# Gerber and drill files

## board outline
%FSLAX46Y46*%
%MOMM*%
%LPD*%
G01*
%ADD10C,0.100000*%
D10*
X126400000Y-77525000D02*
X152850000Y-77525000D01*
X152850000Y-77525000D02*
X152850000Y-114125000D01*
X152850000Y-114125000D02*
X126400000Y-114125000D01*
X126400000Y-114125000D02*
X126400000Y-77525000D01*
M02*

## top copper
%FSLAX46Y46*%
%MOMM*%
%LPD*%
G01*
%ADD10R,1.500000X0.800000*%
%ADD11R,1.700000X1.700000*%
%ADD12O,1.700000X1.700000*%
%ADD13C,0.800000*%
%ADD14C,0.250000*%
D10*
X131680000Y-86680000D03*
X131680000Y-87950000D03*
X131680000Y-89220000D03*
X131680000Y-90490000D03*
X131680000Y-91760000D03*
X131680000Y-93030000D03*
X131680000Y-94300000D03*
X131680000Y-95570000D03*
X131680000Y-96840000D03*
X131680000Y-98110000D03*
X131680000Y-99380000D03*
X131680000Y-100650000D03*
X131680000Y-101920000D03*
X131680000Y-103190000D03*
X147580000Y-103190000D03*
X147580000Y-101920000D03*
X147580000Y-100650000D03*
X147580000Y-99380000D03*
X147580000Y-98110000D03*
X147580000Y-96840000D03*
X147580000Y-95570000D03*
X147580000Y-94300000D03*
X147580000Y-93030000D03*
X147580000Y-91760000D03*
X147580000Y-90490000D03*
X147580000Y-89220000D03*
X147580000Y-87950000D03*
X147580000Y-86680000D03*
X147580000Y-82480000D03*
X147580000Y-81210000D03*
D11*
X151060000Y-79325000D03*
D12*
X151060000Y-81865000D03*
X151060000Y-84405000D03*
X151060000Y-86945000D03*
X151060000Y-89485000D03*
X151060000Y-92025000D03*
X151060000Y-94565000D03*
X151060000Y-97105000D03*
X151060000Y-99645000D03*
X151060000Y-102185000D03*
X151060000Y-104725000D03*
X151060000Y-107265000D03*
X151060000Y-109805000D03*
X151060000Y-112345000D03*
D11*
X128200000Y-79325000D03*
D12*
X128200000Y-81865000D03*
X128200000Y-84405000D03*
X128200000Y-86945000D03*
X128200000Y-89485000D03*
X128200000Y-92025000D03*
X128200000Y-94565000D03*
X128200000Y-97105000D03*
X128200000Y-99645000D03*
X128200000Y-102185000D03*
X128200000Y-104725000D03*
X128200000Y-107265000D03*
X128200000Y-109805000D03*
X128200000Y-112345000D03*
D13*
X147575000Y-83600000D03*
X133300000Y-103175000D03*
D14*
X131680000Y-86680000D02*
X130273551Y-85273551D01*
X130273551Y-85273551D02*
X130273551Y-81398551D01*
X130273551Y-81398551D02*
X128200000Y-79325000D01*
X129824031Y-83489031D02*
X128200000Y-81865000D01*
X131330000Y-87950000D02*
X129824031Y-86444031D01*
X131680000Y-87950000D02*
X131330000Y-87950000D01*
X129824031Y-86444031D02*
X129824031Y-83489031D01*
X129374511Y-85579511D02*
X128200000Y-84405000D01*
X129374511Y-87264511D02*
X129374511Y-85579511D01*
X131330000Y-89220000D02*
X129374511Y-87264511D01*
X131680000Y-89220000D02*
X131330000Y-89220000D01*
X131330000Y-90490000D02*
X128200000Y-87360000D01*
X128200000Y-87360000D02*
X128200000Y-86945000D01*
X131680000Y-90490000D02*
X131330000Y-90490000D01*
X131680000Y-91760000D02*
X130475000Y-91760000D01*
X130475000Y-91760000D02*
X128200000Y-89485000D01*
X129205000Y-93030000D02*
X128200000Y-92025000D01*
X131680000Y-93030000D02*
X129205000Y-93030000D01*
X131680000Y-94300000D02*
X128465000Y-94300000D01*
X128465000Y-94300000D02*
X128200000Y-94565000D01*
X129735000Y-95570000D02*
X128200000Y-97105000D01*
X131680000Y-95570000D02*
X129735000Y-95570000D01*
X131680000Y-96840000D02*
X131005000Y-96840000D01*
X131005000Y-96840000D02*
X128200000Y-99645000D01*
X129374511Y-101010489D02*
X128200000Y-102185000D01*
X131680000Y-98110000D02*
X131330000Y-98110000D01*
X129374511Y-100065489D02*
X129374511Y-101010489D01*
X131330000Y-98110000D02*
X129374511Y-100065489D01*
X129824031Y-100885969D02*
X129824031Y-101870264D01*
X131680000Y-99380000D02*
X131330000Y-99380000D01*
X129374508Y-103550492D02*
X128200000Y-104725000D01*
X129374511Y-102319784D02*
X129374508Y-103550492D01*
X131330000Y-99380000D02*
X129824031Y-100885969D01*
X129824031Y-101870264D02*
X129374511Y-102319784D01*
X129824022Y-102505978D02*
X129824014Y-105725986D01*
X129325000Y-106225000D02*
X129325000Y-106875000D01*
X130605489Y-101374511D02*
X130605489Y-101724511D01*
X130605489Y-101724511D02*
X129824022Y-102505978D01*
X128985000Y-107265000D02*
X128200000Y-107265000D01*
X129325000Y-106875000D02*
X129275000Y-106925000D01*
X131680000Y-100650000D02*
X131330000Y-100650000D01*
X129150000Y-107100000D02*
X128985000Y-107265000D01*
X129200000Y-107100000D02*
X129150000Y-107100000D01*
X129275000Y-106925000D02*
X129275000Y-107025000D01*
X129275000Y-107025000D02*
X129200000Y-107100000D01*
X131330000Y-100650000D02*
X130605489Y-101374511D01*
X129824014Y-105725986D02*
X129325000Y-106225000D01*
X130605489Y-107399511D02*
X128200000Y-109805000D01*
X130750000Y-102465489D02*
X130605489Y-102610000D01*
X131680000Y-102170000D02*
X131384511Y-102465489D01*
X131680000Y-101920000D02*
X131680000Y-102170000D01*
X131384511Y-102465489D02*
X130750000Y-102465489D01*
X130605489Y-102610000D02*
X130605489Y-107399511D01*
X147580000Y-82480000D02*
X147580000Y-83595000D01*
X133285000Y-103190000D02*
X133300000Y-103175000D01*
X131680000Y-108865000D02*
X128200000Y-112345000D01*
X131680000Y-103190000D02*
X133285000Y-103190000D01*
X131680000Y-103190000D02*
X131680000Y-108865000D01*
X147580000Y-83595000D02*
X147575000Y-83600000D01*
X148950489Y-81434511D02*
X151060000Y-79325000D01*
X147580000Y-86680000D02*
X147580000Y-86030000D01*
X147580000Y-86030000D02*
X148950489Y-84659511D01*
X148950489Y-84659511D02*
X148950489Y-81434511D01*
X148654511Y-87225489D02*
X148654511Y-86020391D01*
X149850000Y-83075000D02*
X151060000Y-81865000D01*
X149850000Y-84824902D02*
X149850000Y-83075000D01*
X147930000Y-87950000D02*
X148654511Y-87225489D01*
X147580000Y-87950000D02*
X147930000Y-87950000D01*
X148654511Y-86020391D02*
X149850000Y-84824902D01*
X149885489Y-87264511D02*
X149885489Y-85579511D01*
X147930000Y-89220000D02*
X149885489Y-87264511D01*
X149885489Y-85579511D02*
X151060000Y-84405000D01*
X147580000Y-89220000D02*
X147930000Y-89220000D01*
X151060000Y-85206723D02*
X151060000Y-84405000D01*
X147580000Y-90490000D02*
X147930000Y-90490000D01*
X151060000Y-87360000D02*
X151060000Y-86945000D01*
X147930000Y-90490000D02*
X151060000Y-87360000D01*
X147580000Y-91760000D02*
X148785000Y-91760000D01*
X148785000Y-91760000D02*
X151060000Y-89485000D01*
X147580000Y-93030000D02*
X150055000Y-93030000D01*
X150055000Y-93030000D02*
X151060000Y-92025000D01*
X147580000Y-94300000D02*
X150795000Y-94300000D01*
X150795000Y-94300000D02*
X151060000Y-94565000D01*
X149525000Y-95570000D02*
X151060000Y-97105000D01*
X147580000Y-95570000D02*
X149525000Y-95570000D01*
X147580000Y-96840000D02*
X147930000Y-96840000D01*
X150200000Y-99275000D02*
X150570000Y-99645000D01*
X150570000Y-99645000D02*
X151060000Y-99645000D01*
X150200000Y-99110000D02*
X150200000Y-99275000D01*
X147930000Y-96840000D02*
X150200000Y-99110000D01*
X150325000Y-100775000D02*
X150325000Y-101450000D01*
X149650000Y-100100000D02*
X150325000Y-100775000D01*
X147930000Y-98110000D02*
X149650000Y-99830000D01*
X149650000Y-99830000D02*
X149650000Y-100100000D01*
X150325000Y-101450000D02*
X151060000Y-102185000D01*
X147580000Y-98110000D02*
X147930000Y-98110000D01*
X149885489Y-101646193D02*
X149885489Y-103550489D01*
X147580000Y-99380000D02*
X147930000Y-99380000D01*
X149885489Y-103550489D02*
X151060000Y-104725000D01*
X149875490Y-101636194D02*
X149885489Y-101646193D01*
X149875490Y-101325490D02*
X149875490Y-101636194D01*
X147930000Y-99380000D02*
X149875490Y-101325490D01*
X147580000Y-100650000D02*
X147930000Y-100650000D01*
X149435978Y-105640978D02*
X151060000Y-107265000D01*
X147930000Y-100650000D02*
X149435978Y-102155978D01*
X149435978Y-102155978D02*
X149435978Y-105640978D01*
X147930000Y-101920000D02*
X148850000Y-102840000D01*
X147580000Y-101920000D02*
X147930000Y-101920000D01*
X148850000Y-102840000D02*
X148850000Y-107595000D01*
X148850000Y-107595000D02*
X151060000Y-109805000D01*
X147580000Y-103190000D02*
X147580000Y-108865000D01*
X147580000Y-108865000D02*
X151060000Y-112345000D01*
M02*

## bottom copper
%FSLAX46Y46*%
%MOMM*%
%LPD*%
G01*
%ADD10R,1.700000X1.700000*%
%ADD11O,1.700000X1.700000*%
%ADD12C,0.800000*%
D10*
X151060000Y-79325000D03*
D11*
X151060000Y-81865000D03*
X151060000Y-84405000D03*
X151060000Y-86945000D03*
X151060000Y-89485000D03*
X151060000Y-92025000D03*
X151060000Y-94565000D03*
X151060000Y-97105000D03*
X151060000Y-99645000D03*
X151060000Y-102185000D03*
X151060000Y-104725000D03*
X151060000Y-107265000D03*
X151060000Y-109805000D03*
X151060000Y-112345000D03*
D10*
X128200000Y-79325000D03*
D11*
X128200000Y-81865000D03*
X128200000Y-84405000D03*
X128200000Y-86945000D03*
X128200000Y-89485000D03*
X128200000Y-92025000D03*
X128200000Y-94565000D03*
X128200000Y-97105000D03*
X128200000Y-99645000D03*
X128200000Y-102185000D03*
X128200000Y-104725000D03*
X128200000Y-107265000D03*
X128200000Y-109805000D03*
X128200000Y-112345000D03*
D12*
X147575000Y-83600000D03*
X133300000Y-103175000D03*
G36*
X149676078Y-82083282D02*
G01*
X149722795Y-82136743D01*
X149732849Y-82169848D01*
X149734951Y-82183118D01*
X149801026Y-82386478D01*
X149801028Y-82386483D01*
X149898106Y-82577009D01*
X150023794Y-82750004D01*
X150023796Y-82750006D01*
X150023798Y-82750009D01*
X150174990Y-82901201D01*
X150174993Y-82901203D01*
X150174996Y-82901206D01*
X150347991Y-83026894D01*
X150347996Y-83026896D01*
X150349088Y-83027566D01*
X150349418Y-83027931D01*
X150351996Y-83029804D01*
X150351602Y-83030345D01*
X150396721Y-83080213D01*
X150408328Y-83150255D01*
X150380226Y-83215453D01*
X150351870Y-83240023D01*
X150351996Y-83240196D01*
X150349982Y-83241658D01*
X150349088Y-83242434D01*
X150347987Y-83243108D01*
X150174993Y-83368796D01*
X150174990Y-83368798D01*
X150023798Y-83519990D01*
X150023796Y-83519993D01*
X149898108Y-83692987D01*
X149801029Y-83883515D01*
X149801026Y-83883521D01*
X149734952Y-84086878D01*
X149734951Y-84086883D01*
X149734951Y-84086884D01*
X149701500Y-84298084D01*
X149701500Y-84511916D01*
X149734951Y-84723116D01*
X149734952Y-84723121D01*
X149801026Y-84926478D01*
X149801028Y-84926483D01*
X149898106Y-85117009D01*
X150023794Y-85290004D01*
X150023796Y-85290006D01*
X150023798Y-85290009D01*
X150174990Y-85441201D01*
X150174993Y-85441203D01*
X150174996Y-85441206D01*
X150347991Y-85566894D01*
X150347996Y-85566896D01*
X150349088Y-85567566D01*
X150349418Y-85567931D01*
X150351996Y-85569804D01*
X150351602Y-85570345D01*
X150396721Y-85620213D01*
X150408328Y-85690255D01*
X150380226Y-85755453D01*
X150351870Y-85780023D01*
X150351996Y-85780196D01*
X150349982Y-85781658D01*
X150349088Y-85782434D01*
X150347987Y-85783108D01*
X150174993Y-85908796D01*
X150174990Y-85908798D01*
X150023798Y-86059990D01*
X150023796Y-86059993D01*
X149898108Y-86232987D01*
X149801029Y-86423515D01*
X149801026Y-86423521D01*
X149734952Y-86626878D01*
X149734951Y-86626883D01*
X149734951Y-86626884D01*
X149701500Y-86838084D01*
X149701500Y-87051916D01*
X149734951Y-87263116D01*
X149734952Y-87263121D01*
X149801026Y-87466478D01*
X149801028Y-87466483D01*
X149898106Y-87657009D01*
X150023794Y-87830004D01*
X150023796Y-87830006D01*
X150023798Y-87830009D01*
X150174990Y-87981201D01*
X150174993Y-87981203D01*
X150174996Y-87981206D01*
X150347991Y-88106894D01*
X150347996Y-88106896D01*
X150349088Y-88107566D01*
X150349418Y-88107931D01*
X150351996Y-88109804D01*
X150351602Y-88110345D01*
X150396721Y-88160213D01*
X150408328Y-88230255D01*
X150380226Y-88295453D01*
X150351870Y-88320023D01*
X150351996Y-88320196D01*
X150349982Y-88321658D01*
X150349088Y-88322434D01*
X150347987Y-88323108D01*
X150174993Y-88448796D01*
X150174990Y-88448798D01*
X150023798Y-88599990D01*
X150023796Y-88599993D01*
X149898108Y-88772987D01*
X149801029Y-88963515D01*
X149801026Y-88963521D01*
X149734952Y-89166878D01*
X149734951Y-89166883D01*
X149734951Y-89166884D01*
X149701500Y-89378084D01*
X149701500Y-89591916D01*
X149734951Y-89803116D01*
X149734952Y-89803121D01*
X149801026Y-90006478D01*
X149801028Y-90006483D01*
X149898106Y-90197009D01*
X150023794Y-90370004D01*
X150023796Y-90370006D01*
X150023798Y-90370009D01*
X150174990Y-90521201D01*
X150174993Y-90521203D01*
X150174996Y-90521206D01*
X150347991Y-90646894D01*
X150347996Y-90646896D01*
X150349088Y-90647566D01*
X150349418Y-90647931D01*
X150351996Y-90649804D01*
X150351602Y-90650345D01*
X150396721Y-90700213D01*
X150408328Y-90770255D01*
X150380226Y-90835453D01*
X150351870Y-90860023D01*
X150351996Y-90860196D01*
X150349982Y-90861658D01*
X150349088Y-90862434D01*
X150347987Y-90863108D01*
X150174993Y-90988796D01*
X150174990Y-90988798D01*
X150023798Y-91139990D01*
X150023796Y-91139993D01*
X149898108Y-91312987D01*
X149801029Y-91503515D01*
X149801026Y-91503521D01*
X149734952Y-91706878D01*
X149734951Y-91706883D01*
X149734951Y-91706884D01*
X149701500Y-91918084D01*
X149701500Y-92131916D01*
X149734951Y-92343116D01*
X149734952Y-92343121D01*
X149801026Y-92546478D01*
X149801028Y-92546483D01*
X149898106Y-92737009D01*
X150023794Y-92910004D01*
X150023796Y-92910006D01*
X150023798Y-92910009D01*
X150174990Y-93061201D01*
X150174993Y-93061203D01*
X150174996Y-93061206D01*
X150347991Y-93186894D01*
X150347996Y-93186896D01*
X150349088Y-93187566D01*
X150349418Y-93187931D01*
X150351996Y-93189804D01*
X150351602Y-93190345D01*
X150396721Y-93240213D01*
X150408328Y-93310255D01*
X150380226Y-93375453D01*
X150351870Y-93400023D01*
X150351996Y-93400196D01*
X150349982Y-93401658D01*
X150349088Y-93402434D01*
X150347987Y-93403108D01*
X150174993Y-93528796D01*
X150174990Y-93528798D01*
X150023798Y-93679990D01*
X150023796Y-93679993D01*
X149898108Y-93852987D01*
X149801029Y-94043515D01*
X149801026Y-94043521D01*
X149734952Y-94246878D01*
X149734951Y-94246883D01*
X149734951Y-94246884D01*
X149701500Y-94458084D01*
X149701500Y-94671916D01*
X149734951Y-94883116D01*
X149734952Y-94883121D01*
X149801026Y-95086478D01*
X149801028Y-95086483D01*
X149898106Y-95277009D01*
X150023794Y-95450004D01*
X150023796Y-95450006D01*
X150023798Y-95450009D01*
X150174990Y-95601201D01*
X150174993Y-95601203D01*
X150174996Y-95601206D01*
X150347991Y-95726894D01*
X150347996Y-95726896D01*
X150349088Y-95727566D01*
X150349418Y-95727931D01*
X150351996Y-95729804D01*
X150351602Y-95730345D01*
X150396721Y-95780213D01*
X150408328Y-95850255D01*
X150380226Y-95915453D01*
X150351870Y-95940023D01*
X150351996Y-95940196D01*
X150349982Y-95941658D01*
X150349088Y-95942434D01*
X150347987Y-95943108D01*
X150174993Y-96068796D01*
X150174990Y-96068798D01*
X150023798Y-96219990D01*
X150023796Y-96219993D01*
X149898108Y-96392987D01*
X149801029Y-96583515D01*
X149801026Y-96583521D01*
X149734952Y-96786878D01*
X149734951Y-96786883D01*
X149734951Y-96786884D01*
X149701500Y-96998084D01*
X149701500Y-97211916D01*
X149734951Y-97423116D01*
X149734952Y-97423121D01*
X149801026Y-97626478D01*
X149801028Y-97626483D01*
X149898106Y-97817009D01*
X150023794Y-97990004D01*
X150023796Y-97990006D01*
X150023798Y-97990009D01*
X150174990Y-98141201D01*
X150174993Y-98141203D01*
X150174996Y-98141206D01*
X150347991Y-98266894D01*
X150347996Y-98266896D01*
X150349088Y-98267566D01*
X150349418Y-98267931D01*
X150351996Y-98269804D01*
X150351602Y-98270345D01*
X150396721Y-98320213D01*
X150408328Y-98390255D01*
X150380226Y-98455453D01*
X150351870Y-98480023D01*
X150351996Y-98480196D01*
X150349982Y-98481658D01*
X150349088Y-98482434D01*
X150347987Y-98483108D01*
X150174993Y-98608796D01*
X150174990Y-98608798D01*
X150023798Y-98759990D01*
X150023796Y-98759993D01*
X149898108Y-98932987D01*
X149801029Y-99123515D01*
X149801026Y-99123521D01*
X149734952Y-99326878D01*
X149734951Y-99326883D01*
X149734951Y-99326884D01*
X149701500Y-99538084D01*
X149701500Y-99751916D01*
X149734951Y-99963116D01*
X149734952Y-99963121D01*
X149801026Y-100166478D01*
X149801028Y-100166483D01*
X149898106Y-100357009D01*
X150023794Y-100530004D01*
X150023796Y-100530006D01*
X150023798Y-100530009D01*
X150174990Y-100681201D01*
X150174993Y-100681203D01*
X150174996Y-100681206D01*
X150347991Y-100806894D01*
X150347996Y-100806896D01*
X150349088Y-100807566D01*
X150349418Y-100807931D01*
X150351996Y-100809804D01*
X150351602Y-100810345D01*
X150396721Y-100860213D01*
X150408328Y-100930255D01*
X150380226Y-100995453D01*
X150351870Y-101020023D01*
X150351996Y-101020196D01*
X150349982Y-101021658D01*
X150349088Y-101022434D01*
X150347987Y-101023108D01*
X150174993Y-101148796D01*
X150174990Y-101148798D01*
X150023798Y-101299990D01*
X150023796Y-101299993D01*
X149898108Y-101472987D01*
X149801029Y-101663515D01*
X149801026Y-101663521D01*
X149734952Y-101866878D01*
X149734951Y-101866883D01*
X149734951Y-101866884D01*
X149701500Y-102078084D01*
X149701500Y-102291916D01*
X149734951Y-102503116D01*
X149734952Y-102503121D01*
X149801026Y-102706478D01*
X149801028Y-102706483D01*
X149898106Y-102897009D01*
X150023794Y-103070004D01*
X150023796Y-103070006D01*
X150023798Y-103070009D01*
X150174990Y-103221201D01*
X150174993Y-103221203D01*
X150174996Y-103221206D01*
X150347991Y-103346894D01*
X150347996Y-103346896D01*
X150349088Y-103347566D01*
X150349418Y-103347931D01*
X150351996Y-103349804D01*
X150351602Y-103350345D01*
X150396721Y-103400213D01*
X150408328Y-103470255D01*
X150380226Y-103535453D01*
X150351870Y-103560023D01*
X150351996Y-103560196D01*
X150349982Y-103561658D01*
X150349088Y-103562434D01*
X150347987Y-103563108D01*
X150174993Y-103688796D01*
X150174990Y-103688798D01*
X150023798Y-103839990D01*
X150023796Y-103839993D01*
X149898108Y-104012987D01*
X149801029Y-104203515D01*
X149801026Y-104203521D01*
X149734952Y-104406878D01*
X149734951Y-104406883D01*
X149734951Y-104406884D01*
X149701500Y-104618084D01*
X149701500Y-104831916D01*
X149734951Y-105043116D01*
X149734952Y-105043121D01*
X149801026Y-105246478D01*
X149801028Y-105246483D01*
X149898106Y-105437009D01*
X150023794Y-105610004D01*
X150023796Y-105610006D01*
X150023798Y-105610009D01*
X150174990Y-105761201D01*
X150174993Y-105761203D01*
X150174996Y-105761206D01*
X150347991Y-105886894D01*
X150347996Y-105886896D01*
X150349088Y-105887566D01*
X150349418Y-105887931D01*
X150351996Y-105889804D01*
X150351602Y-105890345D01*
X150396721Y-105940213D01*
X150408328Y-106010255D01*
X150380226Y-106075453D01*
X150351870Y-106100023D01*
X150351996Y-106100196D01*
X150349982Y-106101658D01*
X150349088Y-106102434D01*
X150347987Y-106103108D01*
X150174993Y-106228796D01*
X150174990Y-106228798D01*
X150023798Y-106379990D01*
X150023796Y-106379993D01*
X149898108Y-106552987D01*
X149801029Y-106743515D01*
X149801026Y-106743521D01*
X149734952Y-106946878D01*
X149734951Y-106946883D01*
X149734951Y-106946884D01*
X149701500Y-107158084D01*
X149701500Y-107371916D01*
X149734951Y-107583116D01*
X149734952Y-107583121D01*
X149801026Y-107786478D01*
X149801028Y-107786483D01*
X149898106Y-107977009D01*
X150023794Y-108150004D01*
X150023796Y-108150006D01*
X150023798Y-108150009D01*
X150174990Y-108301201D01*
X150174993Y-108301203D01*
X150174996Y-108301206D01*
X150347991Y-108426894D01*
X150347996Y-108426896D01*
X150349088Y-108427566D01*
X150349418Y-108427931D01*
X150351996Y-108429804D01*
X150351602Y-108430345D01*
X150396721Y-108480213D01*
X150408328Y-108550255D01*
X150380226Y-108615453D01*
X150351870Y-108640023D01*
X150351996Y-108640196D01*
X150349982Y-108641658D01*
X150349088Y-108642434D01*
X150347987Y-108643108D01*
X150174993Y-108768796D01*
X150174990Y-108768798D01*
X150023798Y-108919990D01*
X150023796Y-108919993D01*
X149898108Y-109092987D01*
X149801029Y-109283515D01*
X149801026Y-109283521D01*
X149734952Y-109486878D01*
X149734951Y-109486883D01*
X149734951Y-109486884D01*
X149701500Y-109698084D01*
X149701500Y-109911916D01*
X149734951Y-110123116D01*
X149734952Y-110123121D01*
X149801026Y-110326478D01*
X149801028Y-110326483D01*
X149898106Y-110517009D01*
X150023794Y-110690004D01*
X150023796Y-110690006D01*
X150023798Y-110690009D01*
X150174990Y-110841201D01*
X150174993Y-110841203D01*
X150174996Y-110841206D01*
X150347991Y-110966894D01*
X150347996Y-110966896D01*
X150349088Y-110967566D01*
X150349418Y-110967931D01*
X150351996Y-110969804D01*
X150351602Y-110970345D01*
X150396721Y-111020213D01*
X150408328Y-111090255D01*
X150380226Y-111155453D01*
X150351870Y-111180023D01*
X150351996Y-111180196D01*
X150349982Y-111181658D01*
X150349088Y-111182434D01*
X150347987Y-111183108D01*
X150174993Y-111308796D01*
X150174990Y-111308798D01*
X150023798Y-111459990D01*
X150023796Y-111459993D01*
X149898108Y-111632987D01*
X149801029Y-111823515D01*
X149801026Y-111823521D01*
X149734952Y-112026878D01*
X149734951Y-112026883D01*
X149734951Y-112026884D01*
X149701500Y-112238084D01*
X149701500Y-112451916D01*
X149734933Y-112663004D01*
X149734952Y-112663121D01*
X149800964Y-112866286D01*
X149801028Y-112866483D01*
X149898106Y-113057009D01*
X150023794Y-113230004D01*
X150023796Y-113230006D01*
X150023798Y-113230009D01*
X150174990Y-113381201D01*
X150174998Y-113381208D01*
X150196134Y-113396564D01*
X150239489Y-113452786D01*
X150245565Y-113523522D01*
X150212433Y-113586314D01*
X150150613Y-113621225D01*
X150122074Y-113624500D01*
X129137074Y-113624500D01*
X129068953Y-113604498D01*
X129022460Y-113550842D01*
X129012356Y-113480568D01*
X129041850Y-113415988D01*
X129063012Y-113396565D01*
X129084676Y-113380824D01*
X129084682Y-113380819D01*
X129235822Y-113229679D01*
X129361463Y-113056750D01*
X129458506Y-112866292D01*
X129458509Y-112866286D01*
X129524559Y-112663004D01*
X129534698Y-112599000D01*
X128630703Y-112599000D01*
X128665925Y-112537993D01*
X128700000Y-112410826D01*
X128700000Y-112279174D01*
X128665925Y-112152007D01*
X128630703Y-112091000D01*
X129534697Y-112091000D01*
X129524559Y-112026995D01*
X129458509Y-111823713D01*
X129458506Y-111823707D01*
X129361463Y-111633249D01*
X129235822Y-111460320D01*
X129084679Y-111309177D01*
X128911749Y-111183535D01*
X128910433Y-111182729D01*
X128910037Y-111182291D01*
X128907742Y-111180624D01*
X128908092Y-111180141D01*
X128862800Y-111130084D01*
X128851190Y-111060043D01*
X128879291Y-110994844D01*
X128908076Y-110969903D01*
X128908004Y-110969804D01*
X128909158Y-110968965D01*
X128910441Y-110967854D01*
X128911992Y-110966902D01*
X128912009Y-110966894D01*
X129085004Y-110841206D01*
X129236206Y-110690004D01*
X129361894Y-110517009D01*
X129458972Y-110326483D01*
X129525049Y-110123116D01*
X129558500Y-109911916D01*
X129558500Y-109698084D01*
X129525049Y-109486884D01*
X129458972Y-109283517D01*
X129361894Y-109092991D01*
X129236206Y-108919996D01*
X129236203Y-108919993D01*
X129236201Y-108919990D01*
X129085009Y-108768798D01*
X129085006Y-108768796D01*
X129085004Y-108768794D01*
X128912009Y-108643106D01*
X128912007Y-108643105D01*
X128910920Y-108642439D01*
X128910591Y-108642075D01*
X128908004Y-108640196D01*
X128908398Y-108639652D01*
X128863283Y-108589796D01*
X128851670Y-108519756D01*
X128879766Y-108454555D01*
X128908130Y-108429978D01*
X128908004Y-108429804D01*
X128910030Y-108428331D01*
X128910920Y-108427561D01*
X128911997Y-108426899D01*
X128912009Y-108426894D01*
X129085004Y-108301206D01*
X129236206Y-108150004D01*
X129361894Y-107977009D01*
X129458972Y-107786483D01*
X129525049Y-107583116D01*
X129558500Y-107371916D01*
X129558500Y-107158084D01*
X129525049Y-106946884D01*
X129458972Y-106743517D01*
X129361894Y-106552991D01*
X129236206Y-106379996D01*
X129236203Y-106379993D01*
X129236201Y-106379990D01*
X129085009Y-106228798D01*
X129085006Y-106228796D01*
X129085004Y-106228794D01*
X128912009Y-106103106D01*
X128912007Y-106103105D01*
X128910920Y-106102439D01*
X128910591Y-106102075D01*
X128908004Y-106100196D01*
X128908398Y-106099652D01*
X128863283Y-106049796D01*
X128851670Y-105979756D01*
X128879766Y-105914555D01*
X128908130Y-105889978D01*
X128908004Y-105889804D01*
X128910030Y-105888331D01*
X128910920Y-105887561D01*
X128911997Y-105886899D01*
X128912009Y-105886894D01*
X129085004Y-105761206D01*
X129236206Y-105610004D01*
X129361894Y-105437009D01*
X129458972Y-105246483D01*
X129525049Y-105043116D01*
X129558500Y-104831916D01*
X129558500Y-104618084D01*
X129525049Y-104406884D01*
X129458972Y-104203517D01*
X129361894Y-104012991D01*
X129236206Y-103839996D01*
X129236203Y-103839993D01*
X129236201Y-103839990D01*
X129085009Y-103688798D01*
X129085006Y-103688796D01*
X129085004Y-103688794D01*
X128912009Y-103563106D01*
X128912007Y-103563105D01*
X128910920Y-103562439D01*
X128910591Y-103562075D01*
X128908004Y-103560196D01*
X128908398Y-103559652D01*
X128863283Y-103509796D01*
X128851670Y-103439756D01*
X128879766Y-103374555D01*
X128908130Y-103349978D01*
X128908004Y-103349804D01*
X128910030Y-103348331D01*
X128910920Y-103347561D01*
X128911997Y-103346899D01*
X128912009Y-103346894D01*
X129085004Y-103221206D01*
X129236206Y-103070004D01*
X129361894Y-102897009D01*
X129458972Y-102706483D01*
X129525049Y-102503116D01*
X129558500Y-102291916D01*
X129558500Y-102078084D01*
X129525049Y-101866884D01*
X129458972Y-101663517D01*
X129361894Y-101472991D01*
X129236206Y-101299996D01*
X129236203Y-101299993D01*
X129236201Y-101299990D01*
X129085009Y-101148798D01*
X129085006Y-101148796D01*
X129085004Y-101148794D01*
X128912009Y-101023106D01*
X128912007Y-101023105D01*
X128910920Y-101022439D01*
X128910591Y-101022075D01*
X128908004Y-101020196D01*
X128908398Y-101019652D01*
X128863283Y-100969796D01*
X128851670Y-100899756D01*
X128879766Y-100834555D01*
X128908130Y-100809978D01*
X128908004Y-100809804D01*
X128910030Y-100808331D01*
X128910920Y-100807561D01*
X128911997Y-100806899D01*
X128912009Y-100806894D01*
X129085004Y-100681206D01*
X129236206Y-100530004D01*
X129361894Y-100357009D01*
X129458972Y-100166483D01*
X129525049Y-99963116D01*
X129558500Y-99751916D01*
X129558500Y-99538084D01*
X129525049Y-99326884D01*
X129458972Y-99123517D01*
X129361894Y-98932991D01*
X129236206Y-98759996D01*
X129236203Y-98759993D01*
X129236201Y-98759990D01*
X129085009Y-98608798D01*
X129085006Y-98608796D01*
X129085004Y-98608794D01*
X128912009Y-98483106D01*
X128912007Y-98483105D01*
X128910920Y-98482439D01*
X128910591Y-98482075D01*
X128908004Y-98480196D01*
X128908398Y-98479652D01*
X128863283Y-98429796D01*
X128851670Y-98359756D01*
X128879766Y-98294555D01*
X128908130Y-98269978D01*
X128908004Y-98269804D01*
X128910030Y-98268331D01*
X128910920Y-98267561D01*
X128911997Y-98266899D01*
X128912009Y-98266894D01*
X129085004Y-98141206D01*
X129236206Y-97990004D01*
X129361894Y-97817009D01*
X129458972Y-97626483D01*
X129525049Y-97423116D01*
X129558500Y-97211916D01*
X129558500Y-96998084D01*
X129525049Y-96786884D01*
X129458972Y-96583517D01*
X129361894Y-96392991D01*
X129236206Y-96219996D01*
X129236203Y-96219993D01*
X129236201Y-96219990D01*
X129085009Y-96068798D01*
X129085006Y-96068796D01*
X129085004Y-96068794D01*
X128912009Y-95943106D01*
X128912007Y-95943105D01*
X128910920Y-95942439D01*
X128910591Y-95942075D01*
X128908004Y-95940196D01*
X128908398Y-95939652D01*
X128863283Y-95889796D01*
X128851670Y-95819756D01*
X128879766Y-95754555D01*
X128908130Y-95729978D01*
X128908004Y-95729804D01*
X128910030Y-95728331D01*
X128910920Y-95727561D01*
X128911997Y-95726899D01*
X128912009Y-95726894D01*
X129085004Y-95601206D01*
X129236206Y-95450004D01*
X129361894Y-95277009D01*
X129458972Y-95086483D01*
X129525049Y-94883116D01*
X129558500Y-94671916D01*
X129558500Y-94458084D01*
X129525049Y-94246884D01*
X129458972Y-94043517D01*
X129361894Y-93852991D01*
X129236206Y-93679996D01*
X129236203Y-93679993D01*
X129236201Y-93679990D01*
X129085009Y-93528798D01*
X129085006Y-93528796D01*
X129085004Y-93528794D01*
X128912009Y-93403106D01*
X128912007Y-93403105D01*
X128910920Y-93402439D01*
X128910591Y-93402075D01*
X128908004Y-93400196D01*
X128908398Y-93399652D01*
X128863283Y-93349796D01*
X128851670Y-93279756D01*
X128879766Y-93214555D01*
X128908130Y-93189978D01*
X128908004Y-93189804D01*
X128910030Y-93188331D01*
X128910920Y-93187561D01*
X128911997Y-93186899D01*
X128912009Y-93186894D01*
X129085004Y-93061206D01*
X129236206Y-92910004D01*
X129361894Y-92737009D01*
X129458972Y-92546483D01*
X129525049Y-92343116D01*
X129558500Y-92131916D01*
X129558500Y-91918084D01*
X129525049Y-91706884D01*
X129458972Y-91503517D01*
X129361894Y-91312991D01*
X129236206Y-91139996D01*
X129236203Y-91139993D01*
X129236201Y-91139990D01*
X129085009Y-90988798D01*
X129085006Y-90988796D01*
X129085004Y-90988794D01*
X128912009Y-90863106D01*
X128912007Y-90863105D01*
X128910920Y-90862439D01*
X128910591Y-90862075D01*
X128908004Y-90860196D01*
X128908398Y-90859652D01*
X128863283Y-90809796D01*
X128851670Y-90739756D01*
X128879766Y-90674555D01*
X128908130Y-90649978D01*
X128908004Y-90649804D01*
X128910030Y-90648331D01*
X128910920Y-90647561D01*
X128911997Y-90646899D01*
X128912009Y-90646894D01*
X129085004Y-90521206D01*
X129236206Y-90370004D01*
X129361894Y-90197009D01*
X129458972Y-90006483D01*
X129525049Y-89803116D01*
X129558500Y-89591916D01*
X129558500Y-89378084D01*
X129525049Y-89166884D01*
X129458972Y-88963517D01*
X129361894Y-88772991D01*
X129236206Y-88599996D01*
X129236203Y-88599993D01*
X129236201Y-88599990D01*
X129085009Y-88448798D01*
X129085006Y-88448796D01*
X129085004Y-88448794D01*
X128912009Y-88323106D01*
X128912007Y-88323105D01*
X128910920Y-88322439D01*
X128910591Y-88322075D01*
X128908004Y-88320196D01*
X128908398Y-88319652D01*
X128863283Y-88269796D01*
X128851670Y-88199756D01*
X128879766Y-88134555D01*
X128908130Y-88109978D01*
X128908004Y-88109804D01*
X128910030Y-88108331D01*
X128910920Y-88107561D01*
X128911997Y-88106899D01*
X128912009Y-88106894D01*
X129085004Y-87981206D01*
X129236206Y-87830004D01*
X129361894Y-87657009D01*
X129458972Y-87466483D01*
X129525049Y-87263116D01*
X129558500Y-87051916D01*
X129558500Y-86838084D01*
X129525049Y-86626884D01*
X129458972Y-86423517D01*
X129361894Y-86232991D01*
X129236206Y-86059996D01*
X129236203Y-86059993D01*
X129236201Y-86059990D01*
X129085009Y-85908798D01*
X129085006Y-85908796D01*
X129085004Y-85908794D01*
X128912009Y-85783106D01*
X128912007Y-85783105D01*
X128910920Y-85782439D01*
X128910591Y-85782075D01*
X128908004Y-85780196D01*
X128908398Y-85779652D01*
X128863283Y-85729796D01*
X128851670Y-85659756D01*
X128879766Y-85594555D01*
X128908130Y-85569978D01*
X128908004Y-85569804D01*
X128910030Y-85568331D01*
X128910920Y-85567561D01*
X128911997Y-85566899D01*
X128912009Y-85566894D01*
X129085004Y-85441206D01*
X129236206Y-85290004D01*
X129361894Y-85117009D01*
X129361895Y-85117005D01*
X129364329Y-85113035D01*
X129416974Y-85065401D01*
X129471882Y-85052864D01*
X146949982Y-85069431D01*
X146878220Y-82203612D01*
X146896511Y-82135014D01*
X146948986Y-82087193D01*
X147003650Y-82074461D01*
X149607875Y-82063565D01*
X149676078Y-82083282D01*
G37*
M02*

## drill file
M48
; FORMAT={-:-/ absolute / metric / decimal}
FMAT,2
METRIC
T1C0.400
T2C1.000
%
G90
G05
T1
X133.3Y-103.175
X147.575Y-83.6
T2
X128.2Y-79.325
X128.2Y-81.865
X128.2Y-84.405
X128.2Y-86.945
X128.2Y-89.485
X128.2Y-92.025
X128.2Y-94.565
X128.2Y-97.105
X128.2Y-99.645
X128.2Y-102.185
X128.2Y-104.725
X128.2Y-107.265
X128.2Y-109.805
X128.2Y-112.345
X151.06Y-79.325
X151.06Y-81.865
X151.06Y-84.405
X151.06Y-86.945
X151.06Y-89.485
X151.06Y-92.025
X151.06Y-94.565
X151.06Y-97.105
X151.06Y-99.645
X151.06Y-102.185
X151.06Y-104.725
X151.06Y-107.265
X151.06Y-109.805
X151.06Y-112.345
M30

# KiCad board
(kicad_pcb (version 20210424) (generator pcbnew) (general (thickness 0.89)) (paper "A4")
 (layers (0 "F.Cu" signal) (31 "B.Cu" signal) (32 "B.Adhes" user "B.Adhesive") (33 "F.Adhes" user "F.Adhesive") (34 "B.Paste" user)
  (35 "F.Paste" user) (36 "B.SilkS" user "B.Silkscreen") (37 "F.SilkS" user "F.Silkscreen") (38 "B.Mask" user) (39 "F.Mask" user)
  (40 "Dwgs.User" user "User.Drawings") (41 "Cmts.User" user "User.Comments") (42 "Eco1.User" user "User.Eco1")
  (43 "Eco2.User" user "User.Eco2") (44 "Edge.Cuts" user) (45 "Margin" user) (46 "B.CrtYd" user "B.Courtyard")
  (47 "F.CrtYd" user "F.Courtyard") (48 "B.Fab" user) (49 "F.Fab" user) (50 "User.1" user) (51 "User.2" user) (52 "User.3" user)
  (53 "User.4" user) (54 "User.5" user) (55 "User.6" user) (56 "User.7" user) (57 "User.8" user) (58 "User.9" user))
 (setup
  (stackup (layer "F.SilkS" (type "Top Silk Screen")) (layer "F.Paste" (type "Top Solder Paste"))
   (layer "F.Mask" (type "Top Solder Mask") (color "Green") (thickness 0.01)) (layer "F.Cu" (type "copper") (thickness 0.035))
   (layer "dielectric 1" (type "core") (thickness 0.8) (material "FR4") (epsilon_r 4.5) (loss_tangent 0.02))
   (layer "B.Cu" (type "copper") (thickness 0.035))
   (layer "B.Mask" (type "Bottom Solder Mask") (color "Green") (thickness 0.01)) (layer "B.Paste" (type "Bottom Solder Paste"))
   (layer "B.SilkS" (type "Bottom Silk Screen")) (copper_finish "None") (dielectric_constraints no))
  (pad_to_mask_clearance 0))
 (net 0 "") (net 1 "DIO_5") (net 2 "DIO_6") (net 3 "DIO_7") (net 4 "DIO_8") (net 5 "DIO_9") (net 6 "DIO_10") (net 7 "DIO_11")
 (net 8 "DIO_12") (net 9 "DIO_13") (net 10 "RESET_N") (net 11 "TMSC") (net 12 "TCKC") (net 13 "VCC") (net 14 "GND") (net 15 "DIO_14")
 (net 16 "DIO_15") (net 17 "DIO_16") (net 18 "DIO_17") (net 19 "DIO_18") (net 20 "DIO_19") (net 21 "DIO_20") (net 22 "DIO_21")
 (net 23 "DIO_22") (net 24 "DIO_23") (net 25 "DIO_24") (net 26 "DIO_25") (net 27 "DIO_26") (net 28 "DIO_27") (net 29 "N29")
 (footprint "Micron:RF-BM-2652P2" (layer "F.Cu") (at 139.63 89.68)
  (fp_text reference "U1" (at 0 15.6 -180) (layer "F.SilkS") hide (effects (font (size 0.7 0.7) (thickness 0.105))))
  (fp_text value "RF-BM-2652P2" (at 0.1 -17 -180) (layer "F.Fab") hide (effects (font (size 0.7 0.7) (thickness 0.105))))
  (pad "1" smd rect (at -7.95 -3) (size 1.5 0.8) (layers "F.Cu" "F.Paste" "F.Mask") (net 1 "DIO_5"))
  (pad "2" smd rect (at -7.95 -1.73) (size 1.5 0.8) (layers "F.Cu" "F.Paste" "F.Mask") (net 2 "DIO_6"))
  (pad "3" smd rect (at -7.95 -0.46) (size 1.5 0.8) (layers "F.Cu" "F.Paste" "F.Mask") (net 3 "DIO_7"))
  (pad "4" smd rect (at -7.95 0.81) (size 1.5 0.8) (layers "F.Cu" "F.Paste" "F.Mask") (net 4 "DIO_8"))
  (pad "5" smd rect (at -7.95 2.08) (size 1.5 0.8) (layers "F.Cu" "F.Paste" "F.Mask") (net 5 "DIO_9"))
  (pad "6" smd rect (at -7.95 3.35) (size 1.5 0.8) (layers "F.Cu" "F.Paste" "F.Mask") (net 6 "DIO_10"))
  (pad "7" smd rect (at -7.95 4.62) (size 1.5 0.8) (layers "F.Cu" "F.Paste" "F.Mask") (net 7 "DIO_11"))
  (pad "8" smd rect (at -7.95 5.89) (size 1.5 0.8) (layers "F.Cu" "F.Paste" "F.Mask") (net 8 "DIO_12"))
  (pad "9" smd rect (at -7.95 7.16) (size 1.5 0.8) (layers "F.Cu" "F.Paste" "F.Mask") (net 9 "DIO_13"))
  (pad "10" smd rect (at -7.95 8.43) (size 1.5 0.8) (layers "F.Cu" "F.Paste" "F.Mask") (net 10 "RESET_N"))
  (pad "11" smd rect (at -7.95 9.7) (size 1.5 0.8) (layers "F.Cu" "F.Paste" "F.Mask") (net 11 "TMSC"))
  (pad "12" smd rect (at -7.95 10.97) (size 1.5 0.8) (layers "F.Cu" "F.Paste" "F.Mask") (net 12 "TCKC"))
  (pad "13" smd rect (at -7.95 12.24) (size 1.5 0.8) (layers "F.Cu" "F.Paste" "F.Mask") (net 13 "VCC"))
  (pad "14" smd rect (at -7.95 13.51) (size 1.5 0.8) (layers "F.Cu" "F.Paste" "F.Mask") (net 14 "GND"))
  (pad "15" smd rect (at 7.95 13.51) (size 1.5 0.8) (layers "F.Cu" "F.Paste" "F.Mask") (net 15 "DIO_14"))
  (pad "16" smd rect (at 7.95 12.24) (size 1.5 0.8) (layers "F.Cu" "F.Paste" "F.Mask") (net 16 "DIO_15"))
  (pad "17" smd rect (at 7.95 10.97) (size 1.5 0.8) (layers "F.Cu" "F.Paste" "F.Mask") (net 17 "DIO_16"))
  (pad "18" smd rect (at 7.95 9.7) (size 1.5 0.8) (layers "F.Cu" "F.Paste" "F.Mask") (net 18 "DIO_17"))
  (pad "19" smd rect (at 7.95 8.43) (size 1.5 0.8) (layers "F.Cu" "F.Paste" "F.Mask") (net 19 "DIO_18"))
  (pad "20" smd rect (at 7.95 7.16) (size 1.5 0.8) (layers "F.Cu" "F.Paste" "F.Mask") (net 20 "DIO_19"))
  (pad "21" smd rect (at 7.95 5.89) (size 1.5 0.8) (layers "F.Cu" "F.Paste" "F.Mask") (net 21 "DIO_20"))
  (pad "22" smd rect (at 7.95 4.62) (size 1.5 0.8) (layers "F.Cu" "F.Paste" "F.Mask") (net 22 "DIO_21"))
  (pad "23" smd rect (at 7.95 3.35) (size 1.5 0.8) (layers "F.Cu" "F.Paste" "F.Mask") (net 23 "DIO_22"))
  (pad "24" smd rect (at 7.95 2.08) (size 1.5 0.8) (layers "F.Cu" "F.Paste" "F.Mask") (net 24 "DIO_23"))
  (pad "25" smd rect (at 7.95 0.81) (size 1.5 0.8) (layers "F.Cu" "F.Paste" "F.Mask") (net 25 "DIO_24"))
  (pad "26" smd rect (at 7.95 -0.46) (size 1.5 0.8) (layers "F.Cu" "F.Paste" "F.Mask") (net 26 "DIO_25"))
  (pad "27" smd rect (at 7.95 -1.73) (size 1.5 0.8) (layers "F.Cu" "F.Paste" "F.Mask") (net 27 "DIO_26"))
  (pad "28" smd rect (at 7.95 -3) (size 1.5 0.8) (layers "F.Cu" "F.Paste" "F.Mask") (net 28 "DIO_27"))
  (pad "29" smd rect (at 7.95 -7.2) (size 1.5 0.8) (layers "F.Cu" "F.Paste" "F.Mask") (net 14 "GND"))
  (pad "30" smd rect (at 7.95 -8.47) (size 1.5 0.8) (layers "F.Cu" "F.Paste" "F.Mask") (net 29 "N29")))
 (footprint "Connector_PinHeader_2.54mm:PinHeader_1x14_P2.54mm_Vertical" (layer "B.Cu") (at 151.06 79.325 180)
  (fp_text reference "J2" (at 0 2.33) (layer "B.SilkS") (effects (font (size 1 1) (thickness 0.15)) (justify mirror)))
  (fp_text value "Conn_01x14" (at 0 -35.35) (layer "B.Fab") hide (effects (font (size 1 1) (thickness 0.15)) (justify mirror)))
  (pad "1" thru_hole rect locked (at 0 0 180) (size 1.7 1.7) (drill 1) (layers *.Cu *.Mask) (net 28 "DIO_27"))
  (pad "2" thru_hole oval locked (at 0 -2.54 180) (size 1.7 1.7) (drill 1) (layers *.Cu *.Mask) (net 27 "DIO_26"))
  (pad "3" thru_hole oval locked (at 0 -5.08 180) (size 1.7 1.7) (drill 1) (layers *.Cu *.Mask) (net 26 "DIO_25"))
  (pad "4" thru_hole oval locked (at 0 -7.62 180) (size 1.7 1.7) (drill 1) (layers *.Cu *.Mask) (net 25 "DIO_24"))
  (pad "5" thru_hole oval locked (at 0 -10.16 180) (size 1.7 1.7) (drill 1) (layers *.Cu *.Mask) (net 24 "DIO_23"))
  (pad "6" thru_hole oval locked (at 0 -12.7 180) (size 1.7 1.7) (drill 1) (layers *.Cu *.Mask) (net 23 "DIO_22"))
  (pad "7" thru_hole oval locked (at 0 -15.24 180) (size 1.7 1.7) (drill 1) (layers *.Cu *.Mask) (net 22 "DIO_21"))
  (pad "8" thru_hole oval locked (at 0 -17.78 180) (size 1.7 1.7) (drill 1) (layers *.Cu *.Mask) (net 21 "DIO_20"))
  (pad "9" thru_hole oval locked (at 0 -20.32 180) (size 1.7 1.7) (drill 1) (layers *.Cu *.Mask) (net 20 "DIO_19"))
  (pad "10" thru_hole oval locked (at 0 -22.86 180) (size 1.7 1.7) (drill 1) (layers *.Cu *.Mask) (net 19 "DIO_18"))
  (pad "11" thru_hole oval locked (at 0 -25.4 180) (size 1.7 1.7) (drill 1) (layers *.Cu *.Mask) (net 18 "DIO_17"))
  (pad "12" thru_hole oval locked (at 0 -27.94 180) (size 1.7 1.7) (drill 1) (layers *.Cu *.Mask) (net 17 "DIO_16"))
  (pad "13" thru_hole oval locked (at 0 -30.48 180) (size 1.7 1.7) (drill 1) (layers *.Cu *.Mask) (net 16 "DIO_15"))
  (pad "14" thru_hole oval locked (at 0 -33.02 180) (size 1.7 1.7) (drill 1) (layers *.Cu *.Mask) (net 15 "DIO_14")))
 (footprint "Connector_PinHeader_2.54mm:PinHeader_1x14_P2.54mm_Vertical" (layer "B.Cu") (at 128.2 79.325 180)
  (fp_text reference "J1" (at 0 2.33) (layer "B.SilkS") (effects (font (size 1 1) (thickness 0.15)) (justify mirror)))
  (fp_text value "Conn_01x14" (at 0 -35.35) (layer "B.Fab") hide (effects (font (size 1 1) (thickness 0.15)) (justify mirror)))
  (pad "1" thru_hole rect locked (at 0 0 180) (size 1.7 1.7) (drill 1) (layers *.Cu *.Mask) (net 1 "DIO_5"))
  (pad "2" thru_hole oval locked (at 0 -2.54 180) (size 1.7 1.7) (drill 1) (layers *.Cu *.Mask) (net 2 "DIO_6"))
  (pad "3" thru_hole oval locked (at 0 -5.08 180) (size 1.7 1.7) (drill 1) (layers *.Cu *.Mask) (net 3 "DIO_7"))
  (pad "4" thru_hole oval locked (at 0 -7.62 180) (size 1.7 1.7) (drill 1) (layers *.Cu *.Mask) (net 4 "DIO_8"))
  (pad "5" thru_hole oval locked (at 0 -10.16 180) (size 1.7 1.7) (drill 1) (layers *.Cu *.Mask) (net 5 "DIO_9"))
  (pad "6" thru_hole oval locked (at 0 -12.7 180) (size 1.7 1.7) (drill 1) (layers *.Cu *.Mask) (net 6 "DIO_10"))
  (pad "7" thru_hole oval locked (at 0 -15.24 180) (size 1.7 1.7) (drill 1) (layers *.Cu *.Mask) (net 7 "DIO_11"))
  (pad "8" thru_hole oval locked (at 0 -17.78 180) (size 1.7 1.7) (drill 1) (layers *.Cu *.Mask) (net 8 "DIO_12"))
  (pad "9" thru_hole oval locked (at 0 -20.32 180) (size 1.7 1.7) (drill 1) (layers *.Cu *.Mask) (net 9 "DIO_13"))
  (pad "10" thru_hole oval locked (at 0 -22.86 180) (size 1.7 1.7) (drill 1) (layers *.Cu *.Mask) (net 10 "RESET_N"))
  (pad "11" thru_hole oval locked (at 0 -25.4 180) (size 1.7 1.7) (drill 1) (layers *.Cu *.Mask) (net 11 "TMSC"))
  (pad "12" thru_hole oval locked (at 0 -27.94 180) (size 1.7 1.7) (drill 1) (layers *.Cu *.Mask) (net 12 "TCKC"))
  (pad "13" thru_hole oval locked (at 0 -30.48 180) (size 1.7 1.7) (drill 1) (layers *.Cu *.Mask) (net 13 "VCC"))
  (pad "14" thru_hole oval locked (at 0 -33.02 180) (size 1.7 1.7) (drill 1) (layers *.Cu *.Mask) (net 14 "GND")))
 (gr_line (start 126.4 77.525) (end 152.85 77.525) (layer "Edge.Cuts") (width 0.1))
 (gr_line (start 152.85 77.525) (end 152.85 114.125) (layer "Edge.Cuts") (width 0.1))
 (gr_line (start 152.85 114.125) (end 126.4 114.125) (layer "Edge.Cuts") (width 0.1))
 (gr_line (start 126.4 114.125) (end 126.4 77.525) (layer "Edge.Cuts") (width 0.1))
 (segment (start 131.68 86.68) (end 130.273551 85.273551) (width 0.25) (layer "F.Cu") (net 1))
 (segment (start 130.273551 85.273551) (end 130.273551 81.398551) (width 0.25) (layer "F.Cu") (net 1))
 (segment (start 130.273551 81.398551) (end 128.2 79.325) (width 0.25) (layer "F.Cu") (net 1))
 (segment (start 129.824031 83.489031) (end 128.2 81.865) (width 0.25) (layer "F.Cu") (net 2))
 (segment (start 131.33 87.95) (end 129.824031 86.444031) (width 0.25) (layer "F.Cu") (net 2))
 (segment (start 131.68 87.95) (end 131.33 87.95) (width 0.25) (layer "F.Cu") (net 2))
 (segment (start 129.824031 86.444031) (end 129.824031 83.489031) (width 0.25) (layer "F.Cu") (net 2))
 (segment (start 129.374511 85.579511) (end 128.2 84.405) (width 0.25) (layer "F.Cu") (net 3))
 (segment (start 129.374511 87.264511) (end 129.374511 85.579511) (width 0.25) (layer "F.Cu") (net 3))
 (segment (start 131.33 89.22) (end 129.374511 87.264511) (width 0.25) (layer "F.Cu") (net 3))
 (segment (start 131.68 89.22) (end 131.33 89.22) (width 0.25) (layer "F.Cu") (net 3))
 (segment (start 131.33 90.49) (end 128.2 87.36) (width 0.25) (layer "F.Cu") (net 4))
 (segment (start 128.2 87.36) (end 128.2 86.945) (width 0.25) (layer "F.Cu") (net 4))
 (segment (start 131.68 90.49) (end 131.33 90.49) (width 0.25) (layer "F.Cu") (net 4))
 (segment (start 131.68 91.76) (end 130.475 91.76) (width 0.25) (layer "F.Cu") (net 5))
 (segment (start 130.475 91.76) (end 128.2 89.485) (width 0.25) (layer "F.Cu") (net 5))
 (segment (start 129.205 93.03) (end 128.2 92.025) (width 0.25) (layer "F.Cu") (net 6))
 (segment (start 131.68 93.03) (end 129.205 93.03) (width 0.25) (layer "F.Cu") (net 6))
 (segment (start 131.68 94.3) (end 128.465 94.3) (width 0.25) (layer "F.Cu") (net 7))
 (segment (start 128.465 94.3) (end 128.2 94.565) (width 0.25) (layer "F.Cu") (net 7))
 (segment (start 129.735 95.57) (end 128.2 97.105) (width 0.25) (layer "F.Cu") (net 8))
 (segment (start 131.68 95.57) (end 129.735 95.57) (width 0.25) (layer "F.Cu") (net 8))
 (segment (start 131.68 96.84) (end 131.005 96.84) (width 0.25) (layer "F.Cu") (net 9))
 (segment (start 131.005 96.84) (end 128.2 99.645) (width 0.25) (layer "F.Cu") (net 9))
 (segment (start 129.374511 101.010489) (end 128.2 102.185) (width 0.25) (layer "F.Cu") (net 10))
 (segment (start 131.68 98.11) (end 131.33 98.11) (width 0.25) (layer "F.Cu") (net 10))
 (segment (start 129.374511 100.065489) (end 129.374511 101.010489) (width 0.25) (layer "F.Cu") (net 10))
 (segment (start 131.33 98.11) (end 129.374511 100.065489) (width 0.25) (layer "F.Cu") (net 10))
 (segment (start 129.824031 100.885969) (end 129.824031 101.870264) (width 0.25) (layer "F.Cu") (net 11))
 (segment (start 131.68 99.38) (end 131.33 99.38) (width 0.25) (layer "F.Cu") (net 11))
 (segment (start 129.374508 103.550492) (end 128.2 104.725) (width 0.25) (layer "F.Cu") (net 11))
 (segment (start 129.374511 102.319784) (end 129.374508 103.550492) (width 0.25) (layer "F.Cu") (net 11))
 (segment (start 131.33 99.38) (end 129.824031 100.885969) (width 0.25) (layer "F.Cu") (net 11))
 (segment (start 129.824031 101.870264) (end 129.374511 102.319784) (width 0.25) (layer "F.Cu") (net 11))
 (segment (start 129.824022 102.505978) (end 129.824014 105.725986) (width 0.25) (layer "F.Cu") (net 12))
 (segment (start 129.325 106.225) (end 129.325 106.875) (width 0.25) (layer "F.Cu") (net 12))
 (segment (start 130.605489 101.374511) (end 130.605489 101.724511) (width 0.25) (layer "F.Cu") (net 12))
 (segment (start 130.605489 101.724511) (end 129.824022 102.505978) (width 0.25) (layer "F.Cu") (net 12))
 (segment (start 128.985 107.265) (end 128.2 107.265) (width 0.25) (layer "F.Cu") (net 12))
 (segment (start 129.325 106.875) (end 129.275 106.925) (width 0.25) (layer "F.Cu") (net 12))
 (segment (start 131.68 100.65) (end 131.33 100.65) (width 0.25) (layer "F.Cu") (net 12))
 (segment (start 129.15 107.1) (end 128.985 107.265) (width 0.25) (layer "F.Cu") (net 12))
 (segment (start 129.2 107.1) (end 129.15 107.1) (width 0.25) (layer "F.Cu") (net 12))
 (segment (start 129.275 106.925) (end 129.275 107.025) (width 0.25) (layer "F.Cu") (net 12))
 (segment (start 129.275 107.025) (end 129.2 107.1) (width 0.25) (layer "F.Cu") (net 12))
 (segment (start 131.33 100.65) (end 130.605489 101.374511) (width 0.25) (layer "F.Cu") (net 12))
 (segment (start 129.824014 105.725986) (end 129.325 106.225) (width 0.25) (layer "F.Cu") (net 12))
 (segment (start 130.605489 107.399511) (end 128.2 109.805) (width 0.25) (layer "F.Cu") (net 13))
 (segment (start 130.75 102.465489) (end 130.605489 102.61) (width 0.25) (layer "F.Cu") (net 13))
 (segment (start 131.68 102.17) (end 131.384511 102.465489) (width 0.25) (layer "F.Cu") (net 13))
 (segment (start 131.68 101.92) (end 131.68 102.17) (width 0.25) (layer "F.Cu") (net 13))
 (segment (start 131.384511 102.465489) (end 130.75 102.465489) (width 0.25) (layer "F.Cu") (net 13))
 (segment (start 130.605489 102.61) (end 130.605489 107.399511) (width 0.25) (layer "F.Cu") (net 13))
 (segment (start 147.58 82.48) (end 147.58 83.595) (width 0.25) (layer "F.Cu") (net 14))
 (segment (start 133.285 103.19) (end 133.3 103.175) (width 0.25) (layer "F.Cu") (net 14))
 (segment (start 131.68 108.865) (end 128.2 112.345) (width 0.25) (layer "F.Cu") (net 14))
 (segment (start 131.68 103.19) (end 133.285 103.19) (width 0.25) (layer "F.Cu") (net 14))
 (segment (start 131.68 103.19) (end 131.68 108.865) (width 0.25) (layer "F.Cu") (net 14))
 (segment (start 147.58 83.595) (end 147.575 83.6) (width 0.25) (layer "F.Cu") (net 14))
 (via (at 147.575 83.6) (size 0.8) (drill 0.4) (layers "F.Cu" "B.Cu") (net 14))
 (via (at 133.3 103.175) (size 0.8) (drill 0.4) (layers "F.Cu" "B.Cu") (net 14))
 (segment (start 148.950489 81.434511) (end 151.06 79.325) (width 0.25) (layer "F.Cu") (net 28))
 (segment (start 147.58 86.68) (end 147.58 86.03) (width 0.25) (layer "F.Cu") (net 28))
 (segment (start 147.58 86.03) (end 148.950489 84.659511) (width 0.25) (layer "F.Cu") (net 28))
 (segment (start 148.950489 84.659511) (end 148.950489 81.434511) (width 0.25) (layer "F.Cu") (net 28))
 (segment (start 148.654511 87.225489) (end 148.654511 86.020391) (width 0.25) (layer "F.Cu") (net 27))
 (segment (start 149.85 83.075) (end 151.06 81.865) (width 0.25) (layer "F.Cu") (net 27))
 (segment (start 149.85 84.824902) (end 149.85 83.075) (width 0.25) (layer "F.Cu") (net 27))
 (segment (start 147.93 87.95) (end 148.654511 87.225489) (width 0.25) (layer "F.Cu") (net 27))
 (segment (start 147.58 87.95) (end 147.93 87.95) (width 0.25) (layer "F.Cu") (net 27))
 (segment (start 148.654511 86.020391) (end 149.85 84.824902) (width 0.25) (layer "F.Cu") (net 27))
 (segment (start 149.885489 87.264511) (end 149.885489 85.579511) (width 0.25) (layer "F.Cu") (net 26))
 (segment (start 147.93 89.22) (end 149.885489 87.264511) (width 0.25) (layer "F.Cu") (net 26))
 (segment (start 149.885489 85.579511) (end 151.06 84.405) (width 0.25) (layer "F.Cu") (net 26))
 (segment (start 147.58 89.22) (end 147.93 89.22) (width 0.25) (layer "F.Cu") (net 26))
 (segment (start 151.06 85.206723) (end 151.06 84.405) (width 0.25) (layer "F.Cu") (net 26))
 (segment (start 147.58 90.49) (end 147.93 90.49) (width 0.25) (layer "F.Cu") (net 25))
 (segment (start 151.06 87.36) (end 151.06 86.945) (width 0.25) (layer "F.Cu") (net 25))
 (segment (start 147.93 90.49) (end 151.06 87.36) (width 0.25) (layer "F.Cu") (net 25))
 (segment (start 147.58 91.76) (end 148.785 91.76) (width 0.25) (layer "F.Cu") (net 24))
 (segment (start 148.785 91.76) (end 151.06 89.485) (width 0.25) (layer "F.Cu") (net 24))
 (segment (start 147.58 93.03) (end 150.055 93.03) (width 0.25) (layer "F.Cu") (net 23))
 (segment (start 150.055 93.03) (end 151.06 92.025) (width 0.25) (layer "F.Cu") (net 23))
 (segment (start 147.58 94.3) (end 150.795 94.3) (width 0.25) (layer "F.Cu") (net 22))
 (segment (start 150.795 94.3) (end 151.06 94.565) (width 0.25) (layer "F.Cu") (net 22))
 (segment (start 149.525 95.57) (end 151.06 97.105) (width 0.25) (layer "F.Cu") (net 21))
 (segment (start 147.58 95.57) (end 149.525 95.57) (width 0.25) (layer "F.Cu") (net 21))
 (segment (start 147.58 96.84) (end 147.93 96.84) (width 0.25) (layer "F.Cu") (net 20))
 (segment (start 150.2 99.275) (end 150.57 99.645) (width 0.25) (layer "F.Cu") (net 20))
 (segment (start 150.57 99.645) (end 151.06 99.645) (width 0.25) (layer "F.Cu") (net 20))
 (segment (start 150.2 99.11) (end 150.2 99.275) (width 0.25) (layer "F.Cu") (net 20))
 (segment (start 147.93 96.84) (end 150.2 99.11) (width 0.25) (layer "F.Cu") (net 20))
 (segment (start 150.325 100.775) (end 150.325 101.45) (width 0.25) (layer "F.Cu") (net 19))
 (segment (start 149.65 100.1) (end 150.325 100.775) (width 0.25) (layer "F.Cu") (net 19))
 (segment (start 147.93 98.11) (end 149.65 99.83) (width 0.25) (layer "F.Cu") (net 19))
 (segment (start 149.65 99.83) (end 149.65 100.1) (width 0.25) (layer "F.Cu") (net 19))
 (segment (start 150.325 101.45) (end 151.06 102.185) (width 0.25) (layer "F.Cu") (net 19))
 (segment (start 147.58 98.11) (end 147.93 98.11) (width 0.25) (layer "F.Cu") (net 19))
 (segment (start 149.885489 101.646193) (end 149.885489 103.550489) (width 0.25) (layer "F.Cu") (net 18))
 (segment (start 147.58 99.38) (end 147.93 99.38) (width 0.25) (layer "F.Cu") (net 18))
 (segment (start 149.885489 103.550489) (end 151.06 104.725) (width 0.25) (layer "F.Cu") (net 18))
 (segment (start 149.87549 101.636194) (end 149.885489 101.646193) (width 0.25) (layer "F.Cu") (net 18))
 (segment (start 149.87549 101.32549) (end 149.87549 101.636194) (width 0.25) (layer "F.Cu") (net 18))
 (segment (start 147.93 99.38) (end 149.87549 101.32549) (width 0.25) (layer "F.Cu") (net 18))
 (segment (start 147.58 100.65) (end 147.93 100.65) (width 0.25) (layer "F.Cu") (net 17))
 (segment (start 149.435978 105.640978) (end 151.06 107.265) (width 0.25) (layer "F.Cu") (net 17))
 (segment (start 147.93 100.65) (end 149.435978 102.155978) (width 0.25) (layer "F.Cu") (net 17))
 (segment (start 149.435978 102.155978) (end 149.435978 105.640978) (width 0.25) (layer "F.Cu") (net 17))
 (segment (start 147.93 101.92) (end 148.85 102.84) (width 0.25) (layer "F.Cu") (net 16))
 (segment (start 147.58 101.92) (end 147.93 101.92) (width 0.25) (layer "F.Cu") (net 16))
 (segment (start 148.85 102.84) (end 148.85 107.595) (width 0.25) (layer "F.Cu") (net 16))
 (segment (start 148.85 107.595) (end 151.06 109.805) (width 0.25) (layer "F.Cu") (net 16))
 (segment (start 147.58 103.19) (end 147.58 108.865) (width 0.25) (layer "F.Cu") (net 15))
 (segment (start 147.58 108.865) (end 151.06 112.345) (width 0.25) (layer "F.Cu") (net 15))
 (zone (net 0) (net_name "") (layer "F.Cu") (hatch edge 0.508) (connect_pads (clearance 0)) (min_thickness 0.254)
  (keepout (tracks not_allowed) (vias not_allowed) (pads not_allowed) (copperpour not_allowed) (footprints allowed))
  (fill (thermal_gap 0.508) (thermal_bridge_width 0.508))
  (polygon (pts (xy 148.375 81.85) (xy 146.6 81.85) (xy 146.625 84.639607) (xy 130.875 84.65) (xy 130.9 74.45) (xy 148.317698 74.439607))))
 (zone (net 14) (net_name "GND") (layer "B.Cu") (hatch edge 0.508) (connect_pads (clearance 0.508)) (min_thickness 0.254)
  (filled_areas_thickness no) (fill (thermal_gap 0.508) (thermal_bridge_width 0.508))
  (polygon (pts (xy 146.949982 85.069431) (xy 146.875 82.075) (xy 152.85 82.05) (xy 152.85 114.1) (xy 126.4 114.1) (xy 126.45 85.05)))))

